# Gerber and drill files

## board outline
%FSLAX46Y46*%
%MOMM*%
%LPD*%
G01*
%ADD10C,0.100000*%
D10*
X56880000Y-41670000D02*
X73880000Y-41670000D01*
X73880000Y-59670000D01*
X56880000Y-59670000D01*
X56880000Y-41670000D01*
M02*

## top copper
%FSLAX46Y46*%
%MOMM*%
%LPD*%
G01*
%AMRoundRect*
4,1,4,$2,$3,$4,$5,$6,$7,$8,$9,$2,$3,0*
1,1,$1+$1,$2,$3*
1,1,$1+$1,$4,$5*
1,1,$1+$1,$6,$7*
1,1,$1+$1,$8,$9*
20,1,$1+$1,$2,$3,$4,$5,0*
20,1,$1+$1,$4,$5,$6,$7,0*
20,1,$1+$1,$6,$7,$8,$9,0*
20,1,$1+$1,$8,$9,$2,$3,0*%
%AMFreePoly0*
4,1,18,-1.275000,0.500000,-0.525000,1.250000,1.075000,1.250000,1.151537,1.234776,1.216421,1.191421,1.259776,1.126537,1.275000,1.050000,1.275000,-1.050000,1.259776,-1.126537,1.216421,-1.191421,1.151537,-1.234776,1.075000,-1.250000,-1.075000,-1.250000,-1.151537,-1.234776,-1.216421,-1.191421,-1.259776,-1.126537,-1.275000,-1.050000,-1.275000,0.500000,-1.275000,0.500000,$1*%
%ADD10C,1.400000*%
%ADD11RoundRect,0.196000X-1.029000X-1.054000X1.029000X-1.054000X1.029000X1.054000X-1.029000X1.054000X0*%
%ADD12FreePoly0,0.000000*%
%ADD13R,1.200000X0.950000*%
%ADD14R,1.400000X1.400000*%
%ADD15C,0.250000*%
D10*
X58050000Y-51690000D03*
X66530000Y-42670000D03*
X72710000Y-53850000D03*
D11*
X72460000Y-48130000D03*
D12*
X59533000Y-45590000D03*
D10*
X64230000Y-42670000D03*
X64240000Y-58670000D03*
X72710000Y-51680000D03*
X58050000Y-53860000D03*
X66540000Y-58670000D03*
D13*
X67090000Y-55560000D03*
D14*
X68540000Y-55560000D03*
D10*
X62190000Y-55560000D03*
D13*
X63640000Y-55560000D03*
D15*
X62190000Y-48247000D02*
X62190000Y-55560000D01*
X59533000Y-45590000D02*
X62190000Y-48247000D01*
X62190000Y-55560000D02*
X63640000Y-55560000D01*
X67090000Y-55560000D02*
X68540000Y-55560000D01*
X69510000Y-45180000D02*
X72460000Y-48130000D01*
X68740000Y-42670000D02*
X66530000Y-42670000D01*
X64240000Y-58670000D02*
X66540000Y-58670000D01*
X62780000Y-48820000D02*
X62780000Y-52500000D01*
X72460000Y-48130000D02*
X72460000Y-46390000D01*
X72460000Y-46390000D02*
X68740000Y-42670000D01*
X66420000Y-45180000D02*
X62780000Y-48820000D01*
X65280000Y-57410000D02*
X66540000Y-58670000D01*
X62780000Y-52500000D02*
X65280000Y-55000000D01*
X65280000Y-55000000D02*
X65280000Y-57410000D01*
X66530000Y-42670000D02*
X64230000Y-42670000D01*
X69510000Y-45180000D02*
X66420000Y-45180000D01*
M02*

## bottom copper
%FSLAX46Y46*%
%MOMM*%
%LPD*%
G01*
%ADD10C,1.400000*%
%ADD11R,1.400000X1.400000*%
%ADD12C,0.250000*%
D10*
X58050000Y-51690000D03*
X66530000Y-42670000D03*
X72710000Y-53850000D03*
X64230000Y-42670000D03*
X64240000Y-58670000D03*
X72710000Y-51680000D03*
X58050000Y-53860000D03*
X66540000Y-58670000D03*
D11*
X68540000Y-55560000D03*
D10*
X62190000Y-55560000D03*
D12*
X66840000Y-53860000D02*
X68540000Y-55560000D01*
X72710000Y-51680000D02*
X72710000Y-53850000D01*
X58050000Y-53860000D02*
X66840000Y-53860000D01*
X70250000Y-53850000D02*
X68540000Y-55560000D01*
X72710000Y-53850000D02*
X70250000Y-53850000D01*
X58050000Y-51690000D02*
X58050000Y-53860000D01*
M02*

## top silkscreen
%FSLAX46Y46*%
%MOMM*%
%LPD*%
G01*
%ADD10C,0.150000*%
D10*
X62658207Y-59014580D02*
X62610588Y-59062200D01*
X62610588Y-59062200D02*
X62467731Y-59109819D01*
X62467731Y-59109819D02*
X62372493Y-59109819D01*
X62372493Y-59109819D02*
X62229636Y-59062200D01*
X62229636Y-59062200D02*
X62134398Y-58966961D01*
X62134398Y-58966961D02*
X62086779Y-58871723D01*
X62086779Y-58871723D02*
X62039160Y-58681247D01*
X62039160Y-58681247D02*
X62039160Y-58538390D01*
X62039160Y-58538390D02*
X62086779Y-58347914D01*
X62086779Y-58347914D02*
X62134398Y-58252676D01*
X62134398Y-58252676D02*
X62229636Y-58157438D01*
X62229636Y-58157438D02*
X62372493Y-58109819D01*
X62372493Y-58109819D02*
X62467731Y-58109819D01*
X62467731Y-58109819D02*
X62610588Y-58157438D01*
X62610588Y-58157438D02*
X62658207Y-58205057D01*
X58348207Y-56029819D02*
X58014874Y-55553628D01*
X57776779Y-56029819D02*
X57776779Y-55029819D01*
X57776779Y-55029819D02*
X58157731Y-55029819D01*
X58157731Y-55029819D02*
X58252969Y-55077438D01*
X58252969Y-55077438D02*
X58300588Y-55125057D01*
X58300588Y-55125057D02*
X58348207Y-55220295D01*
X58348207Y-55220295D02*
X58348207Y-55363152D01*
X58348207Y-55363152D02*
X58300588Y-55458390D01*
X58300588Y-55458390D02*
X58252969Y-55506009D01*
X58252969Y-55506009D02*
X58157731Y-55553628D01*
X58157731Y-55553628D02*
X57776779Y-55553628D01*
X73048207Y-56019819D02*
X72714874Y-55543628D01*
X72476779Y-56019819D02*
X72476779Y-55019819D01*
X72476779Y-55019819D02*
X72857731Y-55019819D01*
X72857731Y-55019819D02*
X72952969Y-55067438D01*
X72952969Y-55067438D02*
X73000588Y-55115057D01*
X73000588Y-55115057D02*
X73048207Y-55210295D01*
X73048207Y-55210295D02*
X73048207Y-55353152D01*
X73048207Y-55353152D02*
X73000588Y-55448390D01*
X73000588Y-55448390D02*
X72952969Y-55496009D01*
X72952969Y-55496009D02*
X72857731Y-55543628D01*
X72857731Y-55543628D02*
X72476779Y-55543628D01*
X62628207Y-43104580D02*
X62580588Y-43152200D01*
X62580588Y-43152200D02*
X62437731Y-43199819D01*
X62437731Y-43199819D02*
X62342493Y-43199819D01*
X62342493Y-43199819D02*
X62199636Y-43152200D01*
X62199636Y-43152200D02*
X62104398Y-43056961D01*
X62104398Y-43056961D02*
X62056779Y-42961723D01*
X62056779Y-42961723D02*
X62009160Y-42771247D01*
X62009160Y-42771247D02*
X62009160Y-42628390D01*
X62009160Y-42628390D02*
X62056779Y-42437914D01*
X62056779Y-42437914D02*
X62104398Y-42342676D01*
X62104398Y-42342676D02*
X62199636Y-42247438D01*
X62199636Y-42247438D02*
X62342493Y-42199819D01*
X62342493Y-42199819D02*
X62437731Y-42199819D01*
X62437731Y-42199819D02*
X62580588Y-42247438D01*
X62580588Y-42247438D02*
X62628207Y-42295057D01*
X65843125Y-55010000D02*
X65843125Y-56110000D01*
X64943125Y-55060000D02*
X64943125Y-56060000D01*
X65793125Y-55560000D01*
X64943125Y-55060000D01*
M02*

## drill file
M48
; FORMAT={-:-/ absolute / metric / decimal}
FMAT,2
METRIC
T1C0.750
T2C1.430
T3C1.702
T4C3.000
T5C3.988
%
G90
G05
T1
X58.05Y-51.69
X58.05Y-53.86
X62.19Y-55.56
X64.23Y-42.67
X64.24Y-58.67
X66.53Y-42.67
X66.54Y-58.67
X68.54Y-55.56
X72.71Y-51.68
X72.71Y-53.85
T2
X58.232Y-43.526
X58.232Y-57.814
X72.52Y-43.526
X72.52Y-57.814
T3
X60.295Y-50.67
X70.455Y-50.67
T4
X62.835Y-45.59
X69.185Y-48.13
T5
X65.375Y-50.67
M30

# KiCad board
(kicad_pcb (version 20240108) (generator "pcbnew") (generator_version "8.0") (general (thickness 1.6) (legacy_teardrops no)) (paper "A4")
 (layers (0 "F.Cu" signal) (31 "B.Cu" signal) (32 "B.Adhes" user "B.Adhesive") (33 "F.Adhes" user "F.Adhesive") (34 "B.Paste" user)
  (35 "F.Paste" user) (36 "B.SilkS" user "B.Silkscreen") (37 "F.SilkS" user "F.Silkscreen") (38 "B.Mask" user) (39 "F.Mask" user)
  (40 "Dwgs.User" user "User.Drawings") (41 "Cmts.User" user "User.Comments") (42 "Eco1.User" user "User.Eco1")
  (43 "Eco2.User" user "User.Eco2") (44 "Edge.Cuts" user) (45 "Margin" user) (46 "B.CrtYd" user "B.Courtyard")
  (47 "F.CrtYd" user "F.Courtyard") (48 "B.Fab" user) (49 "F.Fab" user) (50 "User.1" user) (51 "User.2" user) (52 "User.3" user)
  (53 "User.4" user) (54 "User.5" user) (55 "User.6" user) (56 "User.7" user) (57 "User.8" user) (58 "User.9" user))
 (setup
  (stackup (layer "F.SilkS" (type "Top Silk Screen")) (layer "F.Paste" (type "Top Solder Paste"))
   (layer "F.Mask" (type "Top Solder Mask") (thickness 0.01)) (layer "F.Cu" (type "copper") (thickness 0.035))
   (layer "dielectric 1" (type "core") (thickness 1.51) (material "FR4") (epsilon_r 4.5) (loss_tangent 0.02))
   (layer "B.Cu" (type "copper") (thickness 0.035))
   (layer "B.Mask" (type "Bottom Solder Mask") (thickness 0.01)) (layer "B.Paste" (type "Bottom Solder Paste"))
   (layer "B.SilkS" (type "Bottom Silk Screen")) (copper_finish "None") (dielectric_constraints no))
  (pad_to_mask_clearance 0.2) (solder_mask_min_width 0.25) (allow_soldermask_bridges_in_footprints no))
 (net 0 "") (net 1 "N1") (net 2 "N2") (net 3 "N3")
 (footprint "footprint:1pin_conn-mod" (layer "F.Cu") (at 58.05 51.69)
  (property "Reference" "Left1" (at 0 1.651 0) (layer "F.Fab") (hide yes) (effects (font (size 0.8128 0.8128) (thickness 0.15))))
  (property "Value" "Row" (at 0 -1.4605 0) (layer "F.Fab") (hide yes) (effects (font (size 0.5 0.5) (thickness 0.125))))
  (pad "1" thru_hole circle (at 0 0) (size 1.4 1.4) (drill 0.75) (layers "*.Cu" "*.Mask") (remove_unused_layers no) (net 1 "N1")))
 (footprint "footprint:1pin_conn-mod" (layer "F.Cu") (at 66.53 42.67)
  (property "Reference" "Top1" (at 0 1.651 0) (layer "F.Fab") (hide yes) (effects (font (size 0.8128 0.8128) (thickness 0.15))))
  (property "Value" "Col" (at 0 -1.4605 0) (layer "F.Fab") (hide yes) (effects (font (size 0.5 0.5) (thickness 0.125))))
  (pad "1" thru_hole circle (at 0 0) (size 1.4 1.4) (drill 0.75) (layers "*.Cu" "*.Mask") (remove_unused_layers no) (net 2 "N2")))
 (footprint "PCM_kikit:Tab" (layer "F.Cu") (at 74.12 45.46 180)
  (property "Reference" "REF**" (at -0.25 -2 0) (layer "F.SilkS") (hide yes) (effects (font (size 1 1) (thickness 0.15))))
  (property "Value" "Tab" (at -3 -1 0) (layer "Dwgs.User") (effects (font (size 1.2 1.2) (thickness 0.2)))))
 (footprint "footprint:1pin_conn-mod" (layer "F.Cu") (at 72.71 53.85)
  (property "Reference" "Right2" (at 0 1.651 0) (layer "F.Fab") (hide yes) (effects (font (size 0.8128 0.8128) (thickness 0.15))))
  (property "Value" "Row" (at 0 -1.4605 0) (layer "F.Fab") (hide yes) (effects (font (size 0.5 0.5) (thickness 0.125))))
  (pad "1" thru_hole circle (at 0 0) (size 1.4 1.4) (drill 0.75) (layers "*.Cu" "*.Mask") (remove_unused_layers no) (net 1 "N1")))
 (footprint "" (layer "F.Cu") (at 57.873 43.17)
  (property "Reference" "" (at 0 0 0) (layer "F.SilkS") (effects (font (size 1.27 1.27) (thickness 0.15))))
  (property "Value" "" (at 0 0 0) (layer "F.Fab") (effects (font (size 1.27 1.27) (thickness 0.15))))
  (pad "" np_thru_hole circle (at 0.3595 0.3565) (size 1.43 1.43) (drill 1.43) (layers "F&B.Cu" "*.Mask") (solder_mask_margin 0.1)))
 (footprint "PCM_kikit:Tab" (layer "F.Cu") (at 60.18 59.89 90)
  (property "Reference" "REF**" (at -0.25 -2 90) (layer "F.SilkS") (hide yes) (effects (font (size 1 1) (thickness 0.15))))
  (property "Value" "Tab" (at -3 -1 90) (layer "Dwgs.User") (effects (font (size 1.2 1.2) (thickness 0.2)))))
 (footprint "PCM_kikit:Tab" (layer "F.Cu") (at 74.1 55.99 180)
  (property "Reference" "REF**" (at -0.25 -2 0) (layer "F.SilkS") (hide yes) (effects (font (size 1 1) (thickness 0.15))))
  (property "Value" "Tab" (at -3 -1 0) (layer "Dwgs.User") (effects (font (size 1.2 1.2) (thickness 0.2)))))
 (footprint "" (layer "F.Cu") (at 57.873 57.4575)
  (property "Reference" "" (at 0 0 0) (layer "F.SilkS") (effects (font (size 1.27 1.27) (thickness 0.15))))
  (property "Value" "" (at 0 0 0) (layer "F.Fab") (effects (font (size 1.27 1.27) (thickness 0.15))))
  (pad "" np_thru_hole circle (at 0.3595 0.3565) (size 1.43 1.43) (drill 1.43) (layers "F&B.Cu" "*.Mask") (solder_mask_margin 0.1)))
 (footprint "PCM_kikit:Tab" (layer "F.Cu") (at 56.65 45.42)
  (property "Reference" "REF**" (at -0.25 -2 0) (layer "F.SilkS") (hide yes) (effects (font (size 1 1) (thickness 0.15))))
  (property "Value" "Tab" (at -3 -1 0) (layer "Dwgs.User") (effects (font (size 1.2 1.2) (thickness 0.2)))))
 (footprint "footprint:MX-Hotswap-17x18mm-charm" (layer "F.Cu") (at 65.375 50.67)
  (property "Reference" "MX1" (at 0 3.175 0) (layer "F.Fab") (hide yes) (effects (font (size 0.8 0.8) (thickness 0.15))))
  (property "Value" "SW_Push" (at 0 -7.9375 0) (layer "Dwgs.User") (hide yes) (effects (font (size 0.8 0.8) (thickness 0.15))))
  (pad "" np_thru_hole circle (at -5.08 0 311.901) (size 1.7018 1.7018) (drill 1.7018) (layers "F&B.Cu" "*.Mask") (solder_mask_margin 0.1))
  (pad "" np_thru_hole circle (at -2.54 -5.08) (size 3 3) (drill 3) (layers "F&B.Cu" "*.Mask") (solder_mask_margin 0.1))
  (pad "" np_thru_hole circle (at 0 0) (size 3.9878 3.9878) (drill 3.9878) (layers "F&B.Cu" "*.Mask") (solder_mask_margin 0.1))
  (pad "" np_thru_hole circle (at 3.81 -2.54) (size 3 3) (drill 3) (layers "F&B.Cu" "*.Mask") (solder_mask_margin 0.1))
  (pad "" np_thru_hole circle (at 5.08 0 311.901) (size 1.7018 1.7018) (drill 1.7018) (layers "F&B.Cu" "*.Mask") (solder_mask_margin 0.1))
  (pad "1" smd roundrect (at 7.085 -2.54) (size 2.45 2.5) (layers "F.Cu" "F.Paste" "F.Mask") (roundrect_rratio 0.08) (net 2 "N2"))
  (pad "2" smd roundrect (at -5.842 -5.08) (size 2.55 2.5) (layers "F.Cu" "F.Paste" "F.Mask") (roundrect_rratio 0.08) (chamfer_ratio 0.3)
   (chamfer top_left) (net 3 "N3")))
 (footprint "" (layer "F.Cu") (at 72.1605 57.4575)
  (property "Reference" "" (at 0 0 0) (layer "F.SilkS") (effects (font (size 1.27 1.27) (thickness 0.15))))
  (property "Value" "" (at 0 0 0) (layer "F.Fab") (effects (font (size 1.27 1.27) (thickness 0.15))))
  (pad "" np_thru_hole circle (at 0.3595 0.3565) (size 1.43 1.43) (drill 1.43) (layers "F&B.Cu" "*.Mask") (solder_mask_margin 0.1)))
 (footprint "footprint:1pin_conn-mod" (layer "F.Cu") (at 64.23 42.67)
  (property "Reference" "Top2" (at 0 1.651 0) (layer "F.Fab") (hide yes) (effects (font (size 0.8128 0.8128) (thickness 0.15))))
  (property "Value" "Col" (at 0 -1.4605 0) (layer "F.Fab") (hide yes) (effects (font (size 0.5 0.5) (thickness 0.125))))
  (pad "1" thru_hole circle (at 0 0) (size 1.4 1.4) (drill 0.75) (layers "*.Cu" "*.Mask") (remove_unused_layers no) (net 2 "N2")))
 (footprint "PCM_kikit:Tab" (layer "F.Cu") (at 56.63 55.95)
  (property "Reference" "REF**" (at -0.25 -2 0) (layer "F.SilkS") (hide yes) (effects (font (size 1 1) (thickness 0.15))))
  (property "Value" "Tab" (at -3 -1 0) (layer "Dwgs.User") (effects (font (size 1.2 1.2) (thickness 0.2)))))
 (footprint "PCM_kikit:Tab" (layer "F.Cu") (at 70.75 41.47 -90)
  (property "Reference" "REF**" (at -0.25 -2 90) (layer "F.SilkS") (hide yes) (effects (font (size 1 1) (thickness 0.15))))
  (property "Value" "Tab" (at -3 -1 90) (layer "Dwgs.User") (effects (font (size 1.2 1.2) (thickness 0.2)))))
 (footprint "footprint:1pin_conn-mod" (layer "F.Cu") (at 64.24 58.67)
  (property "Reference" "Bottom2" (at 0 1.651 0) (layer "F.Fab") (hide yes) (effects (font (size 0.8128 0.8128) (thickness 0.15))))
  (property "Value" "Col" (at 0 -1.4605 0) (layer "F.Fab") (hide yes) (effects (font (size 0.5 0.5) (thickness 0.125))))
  (pad "1" thru_hole circle (at 0 0) (size 1.4 1.4) (drill 0.75) (layers "*.Cu" "*.Mask") (remove_unused_layers no) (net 2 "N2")))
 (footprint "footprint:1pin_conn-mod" (layer "F.Cu") (at 72.71 51.68)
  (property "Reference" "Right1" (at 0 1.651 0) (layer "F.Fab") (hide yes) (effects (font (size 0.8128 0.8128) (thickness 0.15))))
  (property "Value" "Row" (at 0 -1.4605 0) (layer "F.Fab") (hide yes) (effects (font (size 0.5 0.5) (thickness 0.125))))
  (pad "1" thru_hole circle (at 0 0) (size 1.4 1.4) (drill 0.75) (layers "*.Cu" "*.Mask") (remove_unused_layers no) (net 1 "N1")))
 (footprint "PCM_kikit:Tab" (layer "F.Cu") (at 70.71 59.91 90)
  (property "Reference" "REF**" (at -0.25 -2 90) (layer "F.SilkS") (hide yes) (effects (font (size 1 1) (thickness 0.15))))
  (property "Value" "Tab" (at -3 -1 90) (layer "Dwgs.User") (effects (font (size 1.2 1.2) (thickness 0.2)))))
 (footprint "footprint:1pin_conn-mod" (layer "F.Cu") (at 58.05 53.86)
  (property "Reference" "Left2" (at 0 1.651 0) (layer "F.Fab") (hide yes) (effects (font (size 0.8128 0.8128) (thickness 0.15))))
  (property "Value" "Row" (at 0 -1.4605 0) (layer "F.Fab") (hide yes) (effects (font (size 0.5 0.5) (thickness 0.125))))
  (pad "1" thru_hole circle (at 0 0) (size 1.4 1.4) (drill 0.75) (layers "*.Cu" "*.Mask") (remove_unused_layers no) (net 1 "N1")))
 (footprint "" (layer "F.Cu") (at 72.1605 43.17)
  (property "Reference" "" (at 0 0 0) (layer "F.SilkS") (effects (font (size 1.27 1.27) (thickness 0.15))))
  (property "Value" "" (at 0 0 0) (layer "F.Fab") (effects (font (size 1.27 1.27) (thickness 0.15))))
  (pad "" np_thru_hole circle (at 0.3595 0.3565) (size 1.43 1.43) (drill 1.43) (layers "F&B.Cu" "*.Mask") (solder_mask_margin 0.1)))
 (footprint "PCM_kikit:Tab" (layer "F.Cu") (at 60.22 41.45 -90)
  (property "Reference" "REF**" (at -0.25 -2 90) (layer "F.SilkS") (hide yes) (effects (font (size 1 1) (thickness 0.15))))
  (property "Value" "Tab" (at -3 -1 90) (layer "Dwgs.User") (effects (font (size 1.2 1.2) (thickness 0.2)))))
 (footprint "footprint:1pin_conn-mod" (layer "F.Cu") (at 66.54 58.67)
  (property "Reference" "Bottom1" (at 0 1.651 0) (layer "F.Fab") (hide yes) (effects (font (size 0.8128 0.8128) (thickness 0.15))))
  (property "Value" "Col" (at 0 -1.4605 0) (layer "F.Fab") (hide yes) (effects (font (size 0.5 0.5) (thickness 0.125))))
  (pad "1" thru_hole circle (at 0 0) (size 1.4 1.4) (drill 0.75) (layers "*.Cu" "*.Mask") (remove_unused_layers no) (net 2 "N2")))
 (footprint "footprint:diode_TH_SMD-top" (layer "F.Cu") (at 68.143125 55.56)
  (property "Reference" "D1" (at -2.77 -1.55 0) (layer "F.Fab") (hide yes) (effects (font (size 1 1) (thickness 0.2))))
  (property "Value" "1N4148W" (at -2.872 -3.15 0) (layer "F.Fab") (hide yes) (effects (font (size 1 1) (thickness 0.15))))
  (fp_line (start -2.3 -0.55) (end -2.3 0.55) (stroke (width 0.15) (type default)) (layer "F.SilkS"))
  (fp_poly (pts (xy -3.2 -0.5) (xy -3.2 0.5) (xy -2.35 0)) (stroke (width 0.15) (type solid)) (fill none) (layer "F.SilkS"))
  (pad "1" smd rect (at -1.053125 0) (size 1.2 0.95) (layers "F.Cu" "F.Paste" "F.Mask") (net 1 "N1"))
  (pad "1" thru_hole rect (at 0.396875 0) (size 1.4 1.4) (drill 0.75) (layers "*.Cu" "*.Mask") (remove_unused_layers no) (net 1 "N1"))
  (pad "2" thru_hole circle (at -5.953125 0) (size 1.4 1.4) (drill 0.75) (layers "*.Cu" "*.Mask") (remove_unused_layers no) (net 3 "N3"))
  (pad "2" smd rect (at -4.503125 0) (size 1.2 0.95) (layers "F.Cu" "F.Paste" "F.Mask") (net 3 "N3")))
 (gr_rect (start 56.88 41.67) (end 73.88 59.67) (stroke (width 0.1) (type default)) (fill none) (layer "Edge.Cuts"))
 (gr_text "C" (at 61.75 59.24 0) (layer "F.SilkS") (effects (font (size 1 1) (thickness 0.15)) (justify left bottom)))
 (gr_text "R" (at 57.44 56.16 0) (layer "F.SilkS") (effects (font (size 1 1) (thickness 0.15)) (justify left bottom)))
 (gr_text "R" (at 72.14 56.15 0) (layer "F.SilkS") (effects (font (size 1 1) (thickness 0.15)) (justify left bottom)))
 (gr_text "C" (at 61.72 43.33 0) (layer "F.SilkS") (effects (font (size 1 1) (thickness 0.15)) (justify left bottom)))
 (segment (start 62.19 48.247) (end 62.19 55.56) (width 0.25) (layer "F.Cu") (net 3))
 (segment (start 59.533 45.59) (end 62.19 48.247) (width 0.25) (layer "F.Cu") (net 3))
 (segment (start 62.19 55.56) (end 63.64 55.56) (width 0.25) (layer "F.Cu") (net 3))
 (segment (start 67.09 55.56) (end 68.54 55.56) (width 0.25) (layer "F.Cu") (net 1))
 (segment (start 66.84 53.86) (end 68.54 55.56) (width 0.25) (layer "B.Cu") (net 1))
 (segment (start 72.71 51.68) (end 72.71 53.85) (width 0.25) (layer "B.Cu") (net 1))
 (segment (start 58.05 53.86) (end 66.84 53.86) (width 0.25) (layer "B.Cu") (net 1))
 (segment (start 70.25 53.85) (end 68.54 55.56) (width 0.25) (layer "B.Cu") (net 1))
 (segment (start 72.71 53.85) (end 70.25 53.85) (width 0.25) (layer "B.Cu") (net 1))
 (segment (start 58.05 51.69) (end 58.05 53.86) (width 0.25) (layer "B.Cu") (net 1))
 (segment (start 69.51 45.18) (end 72.46 48.13) (width 0.25) (layer "F.Cu") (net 2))
 (segment (start 68.74 42.67) (end 66.53 42.67) (width 0.25) (layer "F.Cu") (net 2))
 (segment (start 64.24 58.67) (end 66.54 58.67) (width 0.25) (layer "F.Cu") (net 2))
 (segment (start 62.78 48.82) (end 62.78 52.5) (width 0.25) (layer "F.Cu") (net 2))
 (segment (start 72.46 48.13) (end 72.46 46.39) (width 0.25) (layer "F.Cu") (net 2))
 (segment (start 72.46 46.39) (end 68.74 42.67) (width 0.25) (layer "F.Cu") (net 2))
 (segment (start 66.42 45.18) (end 62.78 48.82) (width 0.25) (layer "F.Cu") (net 2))
 (segment (start 65.28 57.41) (end 66.54 58.67) (width 0.25) (layer "F.Cu") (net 2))
 (segment (start 62.78 52.5) (end 65.28 55) (width 0.25) (layer "F.Cu") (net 2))
 (segment (start 65.28 55) (end 65.28 57.41) (width 0.25) (layer "F.Cu") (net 2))
 (segment (start 66.53 42.67) (end 64.23 42.67) (width 0.25) (layer "F.Cu") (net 2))
 (segment (start 69.51 45.18) (end 66.42 45.18) (width 0.25) (layer "F.Cu") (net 2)))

